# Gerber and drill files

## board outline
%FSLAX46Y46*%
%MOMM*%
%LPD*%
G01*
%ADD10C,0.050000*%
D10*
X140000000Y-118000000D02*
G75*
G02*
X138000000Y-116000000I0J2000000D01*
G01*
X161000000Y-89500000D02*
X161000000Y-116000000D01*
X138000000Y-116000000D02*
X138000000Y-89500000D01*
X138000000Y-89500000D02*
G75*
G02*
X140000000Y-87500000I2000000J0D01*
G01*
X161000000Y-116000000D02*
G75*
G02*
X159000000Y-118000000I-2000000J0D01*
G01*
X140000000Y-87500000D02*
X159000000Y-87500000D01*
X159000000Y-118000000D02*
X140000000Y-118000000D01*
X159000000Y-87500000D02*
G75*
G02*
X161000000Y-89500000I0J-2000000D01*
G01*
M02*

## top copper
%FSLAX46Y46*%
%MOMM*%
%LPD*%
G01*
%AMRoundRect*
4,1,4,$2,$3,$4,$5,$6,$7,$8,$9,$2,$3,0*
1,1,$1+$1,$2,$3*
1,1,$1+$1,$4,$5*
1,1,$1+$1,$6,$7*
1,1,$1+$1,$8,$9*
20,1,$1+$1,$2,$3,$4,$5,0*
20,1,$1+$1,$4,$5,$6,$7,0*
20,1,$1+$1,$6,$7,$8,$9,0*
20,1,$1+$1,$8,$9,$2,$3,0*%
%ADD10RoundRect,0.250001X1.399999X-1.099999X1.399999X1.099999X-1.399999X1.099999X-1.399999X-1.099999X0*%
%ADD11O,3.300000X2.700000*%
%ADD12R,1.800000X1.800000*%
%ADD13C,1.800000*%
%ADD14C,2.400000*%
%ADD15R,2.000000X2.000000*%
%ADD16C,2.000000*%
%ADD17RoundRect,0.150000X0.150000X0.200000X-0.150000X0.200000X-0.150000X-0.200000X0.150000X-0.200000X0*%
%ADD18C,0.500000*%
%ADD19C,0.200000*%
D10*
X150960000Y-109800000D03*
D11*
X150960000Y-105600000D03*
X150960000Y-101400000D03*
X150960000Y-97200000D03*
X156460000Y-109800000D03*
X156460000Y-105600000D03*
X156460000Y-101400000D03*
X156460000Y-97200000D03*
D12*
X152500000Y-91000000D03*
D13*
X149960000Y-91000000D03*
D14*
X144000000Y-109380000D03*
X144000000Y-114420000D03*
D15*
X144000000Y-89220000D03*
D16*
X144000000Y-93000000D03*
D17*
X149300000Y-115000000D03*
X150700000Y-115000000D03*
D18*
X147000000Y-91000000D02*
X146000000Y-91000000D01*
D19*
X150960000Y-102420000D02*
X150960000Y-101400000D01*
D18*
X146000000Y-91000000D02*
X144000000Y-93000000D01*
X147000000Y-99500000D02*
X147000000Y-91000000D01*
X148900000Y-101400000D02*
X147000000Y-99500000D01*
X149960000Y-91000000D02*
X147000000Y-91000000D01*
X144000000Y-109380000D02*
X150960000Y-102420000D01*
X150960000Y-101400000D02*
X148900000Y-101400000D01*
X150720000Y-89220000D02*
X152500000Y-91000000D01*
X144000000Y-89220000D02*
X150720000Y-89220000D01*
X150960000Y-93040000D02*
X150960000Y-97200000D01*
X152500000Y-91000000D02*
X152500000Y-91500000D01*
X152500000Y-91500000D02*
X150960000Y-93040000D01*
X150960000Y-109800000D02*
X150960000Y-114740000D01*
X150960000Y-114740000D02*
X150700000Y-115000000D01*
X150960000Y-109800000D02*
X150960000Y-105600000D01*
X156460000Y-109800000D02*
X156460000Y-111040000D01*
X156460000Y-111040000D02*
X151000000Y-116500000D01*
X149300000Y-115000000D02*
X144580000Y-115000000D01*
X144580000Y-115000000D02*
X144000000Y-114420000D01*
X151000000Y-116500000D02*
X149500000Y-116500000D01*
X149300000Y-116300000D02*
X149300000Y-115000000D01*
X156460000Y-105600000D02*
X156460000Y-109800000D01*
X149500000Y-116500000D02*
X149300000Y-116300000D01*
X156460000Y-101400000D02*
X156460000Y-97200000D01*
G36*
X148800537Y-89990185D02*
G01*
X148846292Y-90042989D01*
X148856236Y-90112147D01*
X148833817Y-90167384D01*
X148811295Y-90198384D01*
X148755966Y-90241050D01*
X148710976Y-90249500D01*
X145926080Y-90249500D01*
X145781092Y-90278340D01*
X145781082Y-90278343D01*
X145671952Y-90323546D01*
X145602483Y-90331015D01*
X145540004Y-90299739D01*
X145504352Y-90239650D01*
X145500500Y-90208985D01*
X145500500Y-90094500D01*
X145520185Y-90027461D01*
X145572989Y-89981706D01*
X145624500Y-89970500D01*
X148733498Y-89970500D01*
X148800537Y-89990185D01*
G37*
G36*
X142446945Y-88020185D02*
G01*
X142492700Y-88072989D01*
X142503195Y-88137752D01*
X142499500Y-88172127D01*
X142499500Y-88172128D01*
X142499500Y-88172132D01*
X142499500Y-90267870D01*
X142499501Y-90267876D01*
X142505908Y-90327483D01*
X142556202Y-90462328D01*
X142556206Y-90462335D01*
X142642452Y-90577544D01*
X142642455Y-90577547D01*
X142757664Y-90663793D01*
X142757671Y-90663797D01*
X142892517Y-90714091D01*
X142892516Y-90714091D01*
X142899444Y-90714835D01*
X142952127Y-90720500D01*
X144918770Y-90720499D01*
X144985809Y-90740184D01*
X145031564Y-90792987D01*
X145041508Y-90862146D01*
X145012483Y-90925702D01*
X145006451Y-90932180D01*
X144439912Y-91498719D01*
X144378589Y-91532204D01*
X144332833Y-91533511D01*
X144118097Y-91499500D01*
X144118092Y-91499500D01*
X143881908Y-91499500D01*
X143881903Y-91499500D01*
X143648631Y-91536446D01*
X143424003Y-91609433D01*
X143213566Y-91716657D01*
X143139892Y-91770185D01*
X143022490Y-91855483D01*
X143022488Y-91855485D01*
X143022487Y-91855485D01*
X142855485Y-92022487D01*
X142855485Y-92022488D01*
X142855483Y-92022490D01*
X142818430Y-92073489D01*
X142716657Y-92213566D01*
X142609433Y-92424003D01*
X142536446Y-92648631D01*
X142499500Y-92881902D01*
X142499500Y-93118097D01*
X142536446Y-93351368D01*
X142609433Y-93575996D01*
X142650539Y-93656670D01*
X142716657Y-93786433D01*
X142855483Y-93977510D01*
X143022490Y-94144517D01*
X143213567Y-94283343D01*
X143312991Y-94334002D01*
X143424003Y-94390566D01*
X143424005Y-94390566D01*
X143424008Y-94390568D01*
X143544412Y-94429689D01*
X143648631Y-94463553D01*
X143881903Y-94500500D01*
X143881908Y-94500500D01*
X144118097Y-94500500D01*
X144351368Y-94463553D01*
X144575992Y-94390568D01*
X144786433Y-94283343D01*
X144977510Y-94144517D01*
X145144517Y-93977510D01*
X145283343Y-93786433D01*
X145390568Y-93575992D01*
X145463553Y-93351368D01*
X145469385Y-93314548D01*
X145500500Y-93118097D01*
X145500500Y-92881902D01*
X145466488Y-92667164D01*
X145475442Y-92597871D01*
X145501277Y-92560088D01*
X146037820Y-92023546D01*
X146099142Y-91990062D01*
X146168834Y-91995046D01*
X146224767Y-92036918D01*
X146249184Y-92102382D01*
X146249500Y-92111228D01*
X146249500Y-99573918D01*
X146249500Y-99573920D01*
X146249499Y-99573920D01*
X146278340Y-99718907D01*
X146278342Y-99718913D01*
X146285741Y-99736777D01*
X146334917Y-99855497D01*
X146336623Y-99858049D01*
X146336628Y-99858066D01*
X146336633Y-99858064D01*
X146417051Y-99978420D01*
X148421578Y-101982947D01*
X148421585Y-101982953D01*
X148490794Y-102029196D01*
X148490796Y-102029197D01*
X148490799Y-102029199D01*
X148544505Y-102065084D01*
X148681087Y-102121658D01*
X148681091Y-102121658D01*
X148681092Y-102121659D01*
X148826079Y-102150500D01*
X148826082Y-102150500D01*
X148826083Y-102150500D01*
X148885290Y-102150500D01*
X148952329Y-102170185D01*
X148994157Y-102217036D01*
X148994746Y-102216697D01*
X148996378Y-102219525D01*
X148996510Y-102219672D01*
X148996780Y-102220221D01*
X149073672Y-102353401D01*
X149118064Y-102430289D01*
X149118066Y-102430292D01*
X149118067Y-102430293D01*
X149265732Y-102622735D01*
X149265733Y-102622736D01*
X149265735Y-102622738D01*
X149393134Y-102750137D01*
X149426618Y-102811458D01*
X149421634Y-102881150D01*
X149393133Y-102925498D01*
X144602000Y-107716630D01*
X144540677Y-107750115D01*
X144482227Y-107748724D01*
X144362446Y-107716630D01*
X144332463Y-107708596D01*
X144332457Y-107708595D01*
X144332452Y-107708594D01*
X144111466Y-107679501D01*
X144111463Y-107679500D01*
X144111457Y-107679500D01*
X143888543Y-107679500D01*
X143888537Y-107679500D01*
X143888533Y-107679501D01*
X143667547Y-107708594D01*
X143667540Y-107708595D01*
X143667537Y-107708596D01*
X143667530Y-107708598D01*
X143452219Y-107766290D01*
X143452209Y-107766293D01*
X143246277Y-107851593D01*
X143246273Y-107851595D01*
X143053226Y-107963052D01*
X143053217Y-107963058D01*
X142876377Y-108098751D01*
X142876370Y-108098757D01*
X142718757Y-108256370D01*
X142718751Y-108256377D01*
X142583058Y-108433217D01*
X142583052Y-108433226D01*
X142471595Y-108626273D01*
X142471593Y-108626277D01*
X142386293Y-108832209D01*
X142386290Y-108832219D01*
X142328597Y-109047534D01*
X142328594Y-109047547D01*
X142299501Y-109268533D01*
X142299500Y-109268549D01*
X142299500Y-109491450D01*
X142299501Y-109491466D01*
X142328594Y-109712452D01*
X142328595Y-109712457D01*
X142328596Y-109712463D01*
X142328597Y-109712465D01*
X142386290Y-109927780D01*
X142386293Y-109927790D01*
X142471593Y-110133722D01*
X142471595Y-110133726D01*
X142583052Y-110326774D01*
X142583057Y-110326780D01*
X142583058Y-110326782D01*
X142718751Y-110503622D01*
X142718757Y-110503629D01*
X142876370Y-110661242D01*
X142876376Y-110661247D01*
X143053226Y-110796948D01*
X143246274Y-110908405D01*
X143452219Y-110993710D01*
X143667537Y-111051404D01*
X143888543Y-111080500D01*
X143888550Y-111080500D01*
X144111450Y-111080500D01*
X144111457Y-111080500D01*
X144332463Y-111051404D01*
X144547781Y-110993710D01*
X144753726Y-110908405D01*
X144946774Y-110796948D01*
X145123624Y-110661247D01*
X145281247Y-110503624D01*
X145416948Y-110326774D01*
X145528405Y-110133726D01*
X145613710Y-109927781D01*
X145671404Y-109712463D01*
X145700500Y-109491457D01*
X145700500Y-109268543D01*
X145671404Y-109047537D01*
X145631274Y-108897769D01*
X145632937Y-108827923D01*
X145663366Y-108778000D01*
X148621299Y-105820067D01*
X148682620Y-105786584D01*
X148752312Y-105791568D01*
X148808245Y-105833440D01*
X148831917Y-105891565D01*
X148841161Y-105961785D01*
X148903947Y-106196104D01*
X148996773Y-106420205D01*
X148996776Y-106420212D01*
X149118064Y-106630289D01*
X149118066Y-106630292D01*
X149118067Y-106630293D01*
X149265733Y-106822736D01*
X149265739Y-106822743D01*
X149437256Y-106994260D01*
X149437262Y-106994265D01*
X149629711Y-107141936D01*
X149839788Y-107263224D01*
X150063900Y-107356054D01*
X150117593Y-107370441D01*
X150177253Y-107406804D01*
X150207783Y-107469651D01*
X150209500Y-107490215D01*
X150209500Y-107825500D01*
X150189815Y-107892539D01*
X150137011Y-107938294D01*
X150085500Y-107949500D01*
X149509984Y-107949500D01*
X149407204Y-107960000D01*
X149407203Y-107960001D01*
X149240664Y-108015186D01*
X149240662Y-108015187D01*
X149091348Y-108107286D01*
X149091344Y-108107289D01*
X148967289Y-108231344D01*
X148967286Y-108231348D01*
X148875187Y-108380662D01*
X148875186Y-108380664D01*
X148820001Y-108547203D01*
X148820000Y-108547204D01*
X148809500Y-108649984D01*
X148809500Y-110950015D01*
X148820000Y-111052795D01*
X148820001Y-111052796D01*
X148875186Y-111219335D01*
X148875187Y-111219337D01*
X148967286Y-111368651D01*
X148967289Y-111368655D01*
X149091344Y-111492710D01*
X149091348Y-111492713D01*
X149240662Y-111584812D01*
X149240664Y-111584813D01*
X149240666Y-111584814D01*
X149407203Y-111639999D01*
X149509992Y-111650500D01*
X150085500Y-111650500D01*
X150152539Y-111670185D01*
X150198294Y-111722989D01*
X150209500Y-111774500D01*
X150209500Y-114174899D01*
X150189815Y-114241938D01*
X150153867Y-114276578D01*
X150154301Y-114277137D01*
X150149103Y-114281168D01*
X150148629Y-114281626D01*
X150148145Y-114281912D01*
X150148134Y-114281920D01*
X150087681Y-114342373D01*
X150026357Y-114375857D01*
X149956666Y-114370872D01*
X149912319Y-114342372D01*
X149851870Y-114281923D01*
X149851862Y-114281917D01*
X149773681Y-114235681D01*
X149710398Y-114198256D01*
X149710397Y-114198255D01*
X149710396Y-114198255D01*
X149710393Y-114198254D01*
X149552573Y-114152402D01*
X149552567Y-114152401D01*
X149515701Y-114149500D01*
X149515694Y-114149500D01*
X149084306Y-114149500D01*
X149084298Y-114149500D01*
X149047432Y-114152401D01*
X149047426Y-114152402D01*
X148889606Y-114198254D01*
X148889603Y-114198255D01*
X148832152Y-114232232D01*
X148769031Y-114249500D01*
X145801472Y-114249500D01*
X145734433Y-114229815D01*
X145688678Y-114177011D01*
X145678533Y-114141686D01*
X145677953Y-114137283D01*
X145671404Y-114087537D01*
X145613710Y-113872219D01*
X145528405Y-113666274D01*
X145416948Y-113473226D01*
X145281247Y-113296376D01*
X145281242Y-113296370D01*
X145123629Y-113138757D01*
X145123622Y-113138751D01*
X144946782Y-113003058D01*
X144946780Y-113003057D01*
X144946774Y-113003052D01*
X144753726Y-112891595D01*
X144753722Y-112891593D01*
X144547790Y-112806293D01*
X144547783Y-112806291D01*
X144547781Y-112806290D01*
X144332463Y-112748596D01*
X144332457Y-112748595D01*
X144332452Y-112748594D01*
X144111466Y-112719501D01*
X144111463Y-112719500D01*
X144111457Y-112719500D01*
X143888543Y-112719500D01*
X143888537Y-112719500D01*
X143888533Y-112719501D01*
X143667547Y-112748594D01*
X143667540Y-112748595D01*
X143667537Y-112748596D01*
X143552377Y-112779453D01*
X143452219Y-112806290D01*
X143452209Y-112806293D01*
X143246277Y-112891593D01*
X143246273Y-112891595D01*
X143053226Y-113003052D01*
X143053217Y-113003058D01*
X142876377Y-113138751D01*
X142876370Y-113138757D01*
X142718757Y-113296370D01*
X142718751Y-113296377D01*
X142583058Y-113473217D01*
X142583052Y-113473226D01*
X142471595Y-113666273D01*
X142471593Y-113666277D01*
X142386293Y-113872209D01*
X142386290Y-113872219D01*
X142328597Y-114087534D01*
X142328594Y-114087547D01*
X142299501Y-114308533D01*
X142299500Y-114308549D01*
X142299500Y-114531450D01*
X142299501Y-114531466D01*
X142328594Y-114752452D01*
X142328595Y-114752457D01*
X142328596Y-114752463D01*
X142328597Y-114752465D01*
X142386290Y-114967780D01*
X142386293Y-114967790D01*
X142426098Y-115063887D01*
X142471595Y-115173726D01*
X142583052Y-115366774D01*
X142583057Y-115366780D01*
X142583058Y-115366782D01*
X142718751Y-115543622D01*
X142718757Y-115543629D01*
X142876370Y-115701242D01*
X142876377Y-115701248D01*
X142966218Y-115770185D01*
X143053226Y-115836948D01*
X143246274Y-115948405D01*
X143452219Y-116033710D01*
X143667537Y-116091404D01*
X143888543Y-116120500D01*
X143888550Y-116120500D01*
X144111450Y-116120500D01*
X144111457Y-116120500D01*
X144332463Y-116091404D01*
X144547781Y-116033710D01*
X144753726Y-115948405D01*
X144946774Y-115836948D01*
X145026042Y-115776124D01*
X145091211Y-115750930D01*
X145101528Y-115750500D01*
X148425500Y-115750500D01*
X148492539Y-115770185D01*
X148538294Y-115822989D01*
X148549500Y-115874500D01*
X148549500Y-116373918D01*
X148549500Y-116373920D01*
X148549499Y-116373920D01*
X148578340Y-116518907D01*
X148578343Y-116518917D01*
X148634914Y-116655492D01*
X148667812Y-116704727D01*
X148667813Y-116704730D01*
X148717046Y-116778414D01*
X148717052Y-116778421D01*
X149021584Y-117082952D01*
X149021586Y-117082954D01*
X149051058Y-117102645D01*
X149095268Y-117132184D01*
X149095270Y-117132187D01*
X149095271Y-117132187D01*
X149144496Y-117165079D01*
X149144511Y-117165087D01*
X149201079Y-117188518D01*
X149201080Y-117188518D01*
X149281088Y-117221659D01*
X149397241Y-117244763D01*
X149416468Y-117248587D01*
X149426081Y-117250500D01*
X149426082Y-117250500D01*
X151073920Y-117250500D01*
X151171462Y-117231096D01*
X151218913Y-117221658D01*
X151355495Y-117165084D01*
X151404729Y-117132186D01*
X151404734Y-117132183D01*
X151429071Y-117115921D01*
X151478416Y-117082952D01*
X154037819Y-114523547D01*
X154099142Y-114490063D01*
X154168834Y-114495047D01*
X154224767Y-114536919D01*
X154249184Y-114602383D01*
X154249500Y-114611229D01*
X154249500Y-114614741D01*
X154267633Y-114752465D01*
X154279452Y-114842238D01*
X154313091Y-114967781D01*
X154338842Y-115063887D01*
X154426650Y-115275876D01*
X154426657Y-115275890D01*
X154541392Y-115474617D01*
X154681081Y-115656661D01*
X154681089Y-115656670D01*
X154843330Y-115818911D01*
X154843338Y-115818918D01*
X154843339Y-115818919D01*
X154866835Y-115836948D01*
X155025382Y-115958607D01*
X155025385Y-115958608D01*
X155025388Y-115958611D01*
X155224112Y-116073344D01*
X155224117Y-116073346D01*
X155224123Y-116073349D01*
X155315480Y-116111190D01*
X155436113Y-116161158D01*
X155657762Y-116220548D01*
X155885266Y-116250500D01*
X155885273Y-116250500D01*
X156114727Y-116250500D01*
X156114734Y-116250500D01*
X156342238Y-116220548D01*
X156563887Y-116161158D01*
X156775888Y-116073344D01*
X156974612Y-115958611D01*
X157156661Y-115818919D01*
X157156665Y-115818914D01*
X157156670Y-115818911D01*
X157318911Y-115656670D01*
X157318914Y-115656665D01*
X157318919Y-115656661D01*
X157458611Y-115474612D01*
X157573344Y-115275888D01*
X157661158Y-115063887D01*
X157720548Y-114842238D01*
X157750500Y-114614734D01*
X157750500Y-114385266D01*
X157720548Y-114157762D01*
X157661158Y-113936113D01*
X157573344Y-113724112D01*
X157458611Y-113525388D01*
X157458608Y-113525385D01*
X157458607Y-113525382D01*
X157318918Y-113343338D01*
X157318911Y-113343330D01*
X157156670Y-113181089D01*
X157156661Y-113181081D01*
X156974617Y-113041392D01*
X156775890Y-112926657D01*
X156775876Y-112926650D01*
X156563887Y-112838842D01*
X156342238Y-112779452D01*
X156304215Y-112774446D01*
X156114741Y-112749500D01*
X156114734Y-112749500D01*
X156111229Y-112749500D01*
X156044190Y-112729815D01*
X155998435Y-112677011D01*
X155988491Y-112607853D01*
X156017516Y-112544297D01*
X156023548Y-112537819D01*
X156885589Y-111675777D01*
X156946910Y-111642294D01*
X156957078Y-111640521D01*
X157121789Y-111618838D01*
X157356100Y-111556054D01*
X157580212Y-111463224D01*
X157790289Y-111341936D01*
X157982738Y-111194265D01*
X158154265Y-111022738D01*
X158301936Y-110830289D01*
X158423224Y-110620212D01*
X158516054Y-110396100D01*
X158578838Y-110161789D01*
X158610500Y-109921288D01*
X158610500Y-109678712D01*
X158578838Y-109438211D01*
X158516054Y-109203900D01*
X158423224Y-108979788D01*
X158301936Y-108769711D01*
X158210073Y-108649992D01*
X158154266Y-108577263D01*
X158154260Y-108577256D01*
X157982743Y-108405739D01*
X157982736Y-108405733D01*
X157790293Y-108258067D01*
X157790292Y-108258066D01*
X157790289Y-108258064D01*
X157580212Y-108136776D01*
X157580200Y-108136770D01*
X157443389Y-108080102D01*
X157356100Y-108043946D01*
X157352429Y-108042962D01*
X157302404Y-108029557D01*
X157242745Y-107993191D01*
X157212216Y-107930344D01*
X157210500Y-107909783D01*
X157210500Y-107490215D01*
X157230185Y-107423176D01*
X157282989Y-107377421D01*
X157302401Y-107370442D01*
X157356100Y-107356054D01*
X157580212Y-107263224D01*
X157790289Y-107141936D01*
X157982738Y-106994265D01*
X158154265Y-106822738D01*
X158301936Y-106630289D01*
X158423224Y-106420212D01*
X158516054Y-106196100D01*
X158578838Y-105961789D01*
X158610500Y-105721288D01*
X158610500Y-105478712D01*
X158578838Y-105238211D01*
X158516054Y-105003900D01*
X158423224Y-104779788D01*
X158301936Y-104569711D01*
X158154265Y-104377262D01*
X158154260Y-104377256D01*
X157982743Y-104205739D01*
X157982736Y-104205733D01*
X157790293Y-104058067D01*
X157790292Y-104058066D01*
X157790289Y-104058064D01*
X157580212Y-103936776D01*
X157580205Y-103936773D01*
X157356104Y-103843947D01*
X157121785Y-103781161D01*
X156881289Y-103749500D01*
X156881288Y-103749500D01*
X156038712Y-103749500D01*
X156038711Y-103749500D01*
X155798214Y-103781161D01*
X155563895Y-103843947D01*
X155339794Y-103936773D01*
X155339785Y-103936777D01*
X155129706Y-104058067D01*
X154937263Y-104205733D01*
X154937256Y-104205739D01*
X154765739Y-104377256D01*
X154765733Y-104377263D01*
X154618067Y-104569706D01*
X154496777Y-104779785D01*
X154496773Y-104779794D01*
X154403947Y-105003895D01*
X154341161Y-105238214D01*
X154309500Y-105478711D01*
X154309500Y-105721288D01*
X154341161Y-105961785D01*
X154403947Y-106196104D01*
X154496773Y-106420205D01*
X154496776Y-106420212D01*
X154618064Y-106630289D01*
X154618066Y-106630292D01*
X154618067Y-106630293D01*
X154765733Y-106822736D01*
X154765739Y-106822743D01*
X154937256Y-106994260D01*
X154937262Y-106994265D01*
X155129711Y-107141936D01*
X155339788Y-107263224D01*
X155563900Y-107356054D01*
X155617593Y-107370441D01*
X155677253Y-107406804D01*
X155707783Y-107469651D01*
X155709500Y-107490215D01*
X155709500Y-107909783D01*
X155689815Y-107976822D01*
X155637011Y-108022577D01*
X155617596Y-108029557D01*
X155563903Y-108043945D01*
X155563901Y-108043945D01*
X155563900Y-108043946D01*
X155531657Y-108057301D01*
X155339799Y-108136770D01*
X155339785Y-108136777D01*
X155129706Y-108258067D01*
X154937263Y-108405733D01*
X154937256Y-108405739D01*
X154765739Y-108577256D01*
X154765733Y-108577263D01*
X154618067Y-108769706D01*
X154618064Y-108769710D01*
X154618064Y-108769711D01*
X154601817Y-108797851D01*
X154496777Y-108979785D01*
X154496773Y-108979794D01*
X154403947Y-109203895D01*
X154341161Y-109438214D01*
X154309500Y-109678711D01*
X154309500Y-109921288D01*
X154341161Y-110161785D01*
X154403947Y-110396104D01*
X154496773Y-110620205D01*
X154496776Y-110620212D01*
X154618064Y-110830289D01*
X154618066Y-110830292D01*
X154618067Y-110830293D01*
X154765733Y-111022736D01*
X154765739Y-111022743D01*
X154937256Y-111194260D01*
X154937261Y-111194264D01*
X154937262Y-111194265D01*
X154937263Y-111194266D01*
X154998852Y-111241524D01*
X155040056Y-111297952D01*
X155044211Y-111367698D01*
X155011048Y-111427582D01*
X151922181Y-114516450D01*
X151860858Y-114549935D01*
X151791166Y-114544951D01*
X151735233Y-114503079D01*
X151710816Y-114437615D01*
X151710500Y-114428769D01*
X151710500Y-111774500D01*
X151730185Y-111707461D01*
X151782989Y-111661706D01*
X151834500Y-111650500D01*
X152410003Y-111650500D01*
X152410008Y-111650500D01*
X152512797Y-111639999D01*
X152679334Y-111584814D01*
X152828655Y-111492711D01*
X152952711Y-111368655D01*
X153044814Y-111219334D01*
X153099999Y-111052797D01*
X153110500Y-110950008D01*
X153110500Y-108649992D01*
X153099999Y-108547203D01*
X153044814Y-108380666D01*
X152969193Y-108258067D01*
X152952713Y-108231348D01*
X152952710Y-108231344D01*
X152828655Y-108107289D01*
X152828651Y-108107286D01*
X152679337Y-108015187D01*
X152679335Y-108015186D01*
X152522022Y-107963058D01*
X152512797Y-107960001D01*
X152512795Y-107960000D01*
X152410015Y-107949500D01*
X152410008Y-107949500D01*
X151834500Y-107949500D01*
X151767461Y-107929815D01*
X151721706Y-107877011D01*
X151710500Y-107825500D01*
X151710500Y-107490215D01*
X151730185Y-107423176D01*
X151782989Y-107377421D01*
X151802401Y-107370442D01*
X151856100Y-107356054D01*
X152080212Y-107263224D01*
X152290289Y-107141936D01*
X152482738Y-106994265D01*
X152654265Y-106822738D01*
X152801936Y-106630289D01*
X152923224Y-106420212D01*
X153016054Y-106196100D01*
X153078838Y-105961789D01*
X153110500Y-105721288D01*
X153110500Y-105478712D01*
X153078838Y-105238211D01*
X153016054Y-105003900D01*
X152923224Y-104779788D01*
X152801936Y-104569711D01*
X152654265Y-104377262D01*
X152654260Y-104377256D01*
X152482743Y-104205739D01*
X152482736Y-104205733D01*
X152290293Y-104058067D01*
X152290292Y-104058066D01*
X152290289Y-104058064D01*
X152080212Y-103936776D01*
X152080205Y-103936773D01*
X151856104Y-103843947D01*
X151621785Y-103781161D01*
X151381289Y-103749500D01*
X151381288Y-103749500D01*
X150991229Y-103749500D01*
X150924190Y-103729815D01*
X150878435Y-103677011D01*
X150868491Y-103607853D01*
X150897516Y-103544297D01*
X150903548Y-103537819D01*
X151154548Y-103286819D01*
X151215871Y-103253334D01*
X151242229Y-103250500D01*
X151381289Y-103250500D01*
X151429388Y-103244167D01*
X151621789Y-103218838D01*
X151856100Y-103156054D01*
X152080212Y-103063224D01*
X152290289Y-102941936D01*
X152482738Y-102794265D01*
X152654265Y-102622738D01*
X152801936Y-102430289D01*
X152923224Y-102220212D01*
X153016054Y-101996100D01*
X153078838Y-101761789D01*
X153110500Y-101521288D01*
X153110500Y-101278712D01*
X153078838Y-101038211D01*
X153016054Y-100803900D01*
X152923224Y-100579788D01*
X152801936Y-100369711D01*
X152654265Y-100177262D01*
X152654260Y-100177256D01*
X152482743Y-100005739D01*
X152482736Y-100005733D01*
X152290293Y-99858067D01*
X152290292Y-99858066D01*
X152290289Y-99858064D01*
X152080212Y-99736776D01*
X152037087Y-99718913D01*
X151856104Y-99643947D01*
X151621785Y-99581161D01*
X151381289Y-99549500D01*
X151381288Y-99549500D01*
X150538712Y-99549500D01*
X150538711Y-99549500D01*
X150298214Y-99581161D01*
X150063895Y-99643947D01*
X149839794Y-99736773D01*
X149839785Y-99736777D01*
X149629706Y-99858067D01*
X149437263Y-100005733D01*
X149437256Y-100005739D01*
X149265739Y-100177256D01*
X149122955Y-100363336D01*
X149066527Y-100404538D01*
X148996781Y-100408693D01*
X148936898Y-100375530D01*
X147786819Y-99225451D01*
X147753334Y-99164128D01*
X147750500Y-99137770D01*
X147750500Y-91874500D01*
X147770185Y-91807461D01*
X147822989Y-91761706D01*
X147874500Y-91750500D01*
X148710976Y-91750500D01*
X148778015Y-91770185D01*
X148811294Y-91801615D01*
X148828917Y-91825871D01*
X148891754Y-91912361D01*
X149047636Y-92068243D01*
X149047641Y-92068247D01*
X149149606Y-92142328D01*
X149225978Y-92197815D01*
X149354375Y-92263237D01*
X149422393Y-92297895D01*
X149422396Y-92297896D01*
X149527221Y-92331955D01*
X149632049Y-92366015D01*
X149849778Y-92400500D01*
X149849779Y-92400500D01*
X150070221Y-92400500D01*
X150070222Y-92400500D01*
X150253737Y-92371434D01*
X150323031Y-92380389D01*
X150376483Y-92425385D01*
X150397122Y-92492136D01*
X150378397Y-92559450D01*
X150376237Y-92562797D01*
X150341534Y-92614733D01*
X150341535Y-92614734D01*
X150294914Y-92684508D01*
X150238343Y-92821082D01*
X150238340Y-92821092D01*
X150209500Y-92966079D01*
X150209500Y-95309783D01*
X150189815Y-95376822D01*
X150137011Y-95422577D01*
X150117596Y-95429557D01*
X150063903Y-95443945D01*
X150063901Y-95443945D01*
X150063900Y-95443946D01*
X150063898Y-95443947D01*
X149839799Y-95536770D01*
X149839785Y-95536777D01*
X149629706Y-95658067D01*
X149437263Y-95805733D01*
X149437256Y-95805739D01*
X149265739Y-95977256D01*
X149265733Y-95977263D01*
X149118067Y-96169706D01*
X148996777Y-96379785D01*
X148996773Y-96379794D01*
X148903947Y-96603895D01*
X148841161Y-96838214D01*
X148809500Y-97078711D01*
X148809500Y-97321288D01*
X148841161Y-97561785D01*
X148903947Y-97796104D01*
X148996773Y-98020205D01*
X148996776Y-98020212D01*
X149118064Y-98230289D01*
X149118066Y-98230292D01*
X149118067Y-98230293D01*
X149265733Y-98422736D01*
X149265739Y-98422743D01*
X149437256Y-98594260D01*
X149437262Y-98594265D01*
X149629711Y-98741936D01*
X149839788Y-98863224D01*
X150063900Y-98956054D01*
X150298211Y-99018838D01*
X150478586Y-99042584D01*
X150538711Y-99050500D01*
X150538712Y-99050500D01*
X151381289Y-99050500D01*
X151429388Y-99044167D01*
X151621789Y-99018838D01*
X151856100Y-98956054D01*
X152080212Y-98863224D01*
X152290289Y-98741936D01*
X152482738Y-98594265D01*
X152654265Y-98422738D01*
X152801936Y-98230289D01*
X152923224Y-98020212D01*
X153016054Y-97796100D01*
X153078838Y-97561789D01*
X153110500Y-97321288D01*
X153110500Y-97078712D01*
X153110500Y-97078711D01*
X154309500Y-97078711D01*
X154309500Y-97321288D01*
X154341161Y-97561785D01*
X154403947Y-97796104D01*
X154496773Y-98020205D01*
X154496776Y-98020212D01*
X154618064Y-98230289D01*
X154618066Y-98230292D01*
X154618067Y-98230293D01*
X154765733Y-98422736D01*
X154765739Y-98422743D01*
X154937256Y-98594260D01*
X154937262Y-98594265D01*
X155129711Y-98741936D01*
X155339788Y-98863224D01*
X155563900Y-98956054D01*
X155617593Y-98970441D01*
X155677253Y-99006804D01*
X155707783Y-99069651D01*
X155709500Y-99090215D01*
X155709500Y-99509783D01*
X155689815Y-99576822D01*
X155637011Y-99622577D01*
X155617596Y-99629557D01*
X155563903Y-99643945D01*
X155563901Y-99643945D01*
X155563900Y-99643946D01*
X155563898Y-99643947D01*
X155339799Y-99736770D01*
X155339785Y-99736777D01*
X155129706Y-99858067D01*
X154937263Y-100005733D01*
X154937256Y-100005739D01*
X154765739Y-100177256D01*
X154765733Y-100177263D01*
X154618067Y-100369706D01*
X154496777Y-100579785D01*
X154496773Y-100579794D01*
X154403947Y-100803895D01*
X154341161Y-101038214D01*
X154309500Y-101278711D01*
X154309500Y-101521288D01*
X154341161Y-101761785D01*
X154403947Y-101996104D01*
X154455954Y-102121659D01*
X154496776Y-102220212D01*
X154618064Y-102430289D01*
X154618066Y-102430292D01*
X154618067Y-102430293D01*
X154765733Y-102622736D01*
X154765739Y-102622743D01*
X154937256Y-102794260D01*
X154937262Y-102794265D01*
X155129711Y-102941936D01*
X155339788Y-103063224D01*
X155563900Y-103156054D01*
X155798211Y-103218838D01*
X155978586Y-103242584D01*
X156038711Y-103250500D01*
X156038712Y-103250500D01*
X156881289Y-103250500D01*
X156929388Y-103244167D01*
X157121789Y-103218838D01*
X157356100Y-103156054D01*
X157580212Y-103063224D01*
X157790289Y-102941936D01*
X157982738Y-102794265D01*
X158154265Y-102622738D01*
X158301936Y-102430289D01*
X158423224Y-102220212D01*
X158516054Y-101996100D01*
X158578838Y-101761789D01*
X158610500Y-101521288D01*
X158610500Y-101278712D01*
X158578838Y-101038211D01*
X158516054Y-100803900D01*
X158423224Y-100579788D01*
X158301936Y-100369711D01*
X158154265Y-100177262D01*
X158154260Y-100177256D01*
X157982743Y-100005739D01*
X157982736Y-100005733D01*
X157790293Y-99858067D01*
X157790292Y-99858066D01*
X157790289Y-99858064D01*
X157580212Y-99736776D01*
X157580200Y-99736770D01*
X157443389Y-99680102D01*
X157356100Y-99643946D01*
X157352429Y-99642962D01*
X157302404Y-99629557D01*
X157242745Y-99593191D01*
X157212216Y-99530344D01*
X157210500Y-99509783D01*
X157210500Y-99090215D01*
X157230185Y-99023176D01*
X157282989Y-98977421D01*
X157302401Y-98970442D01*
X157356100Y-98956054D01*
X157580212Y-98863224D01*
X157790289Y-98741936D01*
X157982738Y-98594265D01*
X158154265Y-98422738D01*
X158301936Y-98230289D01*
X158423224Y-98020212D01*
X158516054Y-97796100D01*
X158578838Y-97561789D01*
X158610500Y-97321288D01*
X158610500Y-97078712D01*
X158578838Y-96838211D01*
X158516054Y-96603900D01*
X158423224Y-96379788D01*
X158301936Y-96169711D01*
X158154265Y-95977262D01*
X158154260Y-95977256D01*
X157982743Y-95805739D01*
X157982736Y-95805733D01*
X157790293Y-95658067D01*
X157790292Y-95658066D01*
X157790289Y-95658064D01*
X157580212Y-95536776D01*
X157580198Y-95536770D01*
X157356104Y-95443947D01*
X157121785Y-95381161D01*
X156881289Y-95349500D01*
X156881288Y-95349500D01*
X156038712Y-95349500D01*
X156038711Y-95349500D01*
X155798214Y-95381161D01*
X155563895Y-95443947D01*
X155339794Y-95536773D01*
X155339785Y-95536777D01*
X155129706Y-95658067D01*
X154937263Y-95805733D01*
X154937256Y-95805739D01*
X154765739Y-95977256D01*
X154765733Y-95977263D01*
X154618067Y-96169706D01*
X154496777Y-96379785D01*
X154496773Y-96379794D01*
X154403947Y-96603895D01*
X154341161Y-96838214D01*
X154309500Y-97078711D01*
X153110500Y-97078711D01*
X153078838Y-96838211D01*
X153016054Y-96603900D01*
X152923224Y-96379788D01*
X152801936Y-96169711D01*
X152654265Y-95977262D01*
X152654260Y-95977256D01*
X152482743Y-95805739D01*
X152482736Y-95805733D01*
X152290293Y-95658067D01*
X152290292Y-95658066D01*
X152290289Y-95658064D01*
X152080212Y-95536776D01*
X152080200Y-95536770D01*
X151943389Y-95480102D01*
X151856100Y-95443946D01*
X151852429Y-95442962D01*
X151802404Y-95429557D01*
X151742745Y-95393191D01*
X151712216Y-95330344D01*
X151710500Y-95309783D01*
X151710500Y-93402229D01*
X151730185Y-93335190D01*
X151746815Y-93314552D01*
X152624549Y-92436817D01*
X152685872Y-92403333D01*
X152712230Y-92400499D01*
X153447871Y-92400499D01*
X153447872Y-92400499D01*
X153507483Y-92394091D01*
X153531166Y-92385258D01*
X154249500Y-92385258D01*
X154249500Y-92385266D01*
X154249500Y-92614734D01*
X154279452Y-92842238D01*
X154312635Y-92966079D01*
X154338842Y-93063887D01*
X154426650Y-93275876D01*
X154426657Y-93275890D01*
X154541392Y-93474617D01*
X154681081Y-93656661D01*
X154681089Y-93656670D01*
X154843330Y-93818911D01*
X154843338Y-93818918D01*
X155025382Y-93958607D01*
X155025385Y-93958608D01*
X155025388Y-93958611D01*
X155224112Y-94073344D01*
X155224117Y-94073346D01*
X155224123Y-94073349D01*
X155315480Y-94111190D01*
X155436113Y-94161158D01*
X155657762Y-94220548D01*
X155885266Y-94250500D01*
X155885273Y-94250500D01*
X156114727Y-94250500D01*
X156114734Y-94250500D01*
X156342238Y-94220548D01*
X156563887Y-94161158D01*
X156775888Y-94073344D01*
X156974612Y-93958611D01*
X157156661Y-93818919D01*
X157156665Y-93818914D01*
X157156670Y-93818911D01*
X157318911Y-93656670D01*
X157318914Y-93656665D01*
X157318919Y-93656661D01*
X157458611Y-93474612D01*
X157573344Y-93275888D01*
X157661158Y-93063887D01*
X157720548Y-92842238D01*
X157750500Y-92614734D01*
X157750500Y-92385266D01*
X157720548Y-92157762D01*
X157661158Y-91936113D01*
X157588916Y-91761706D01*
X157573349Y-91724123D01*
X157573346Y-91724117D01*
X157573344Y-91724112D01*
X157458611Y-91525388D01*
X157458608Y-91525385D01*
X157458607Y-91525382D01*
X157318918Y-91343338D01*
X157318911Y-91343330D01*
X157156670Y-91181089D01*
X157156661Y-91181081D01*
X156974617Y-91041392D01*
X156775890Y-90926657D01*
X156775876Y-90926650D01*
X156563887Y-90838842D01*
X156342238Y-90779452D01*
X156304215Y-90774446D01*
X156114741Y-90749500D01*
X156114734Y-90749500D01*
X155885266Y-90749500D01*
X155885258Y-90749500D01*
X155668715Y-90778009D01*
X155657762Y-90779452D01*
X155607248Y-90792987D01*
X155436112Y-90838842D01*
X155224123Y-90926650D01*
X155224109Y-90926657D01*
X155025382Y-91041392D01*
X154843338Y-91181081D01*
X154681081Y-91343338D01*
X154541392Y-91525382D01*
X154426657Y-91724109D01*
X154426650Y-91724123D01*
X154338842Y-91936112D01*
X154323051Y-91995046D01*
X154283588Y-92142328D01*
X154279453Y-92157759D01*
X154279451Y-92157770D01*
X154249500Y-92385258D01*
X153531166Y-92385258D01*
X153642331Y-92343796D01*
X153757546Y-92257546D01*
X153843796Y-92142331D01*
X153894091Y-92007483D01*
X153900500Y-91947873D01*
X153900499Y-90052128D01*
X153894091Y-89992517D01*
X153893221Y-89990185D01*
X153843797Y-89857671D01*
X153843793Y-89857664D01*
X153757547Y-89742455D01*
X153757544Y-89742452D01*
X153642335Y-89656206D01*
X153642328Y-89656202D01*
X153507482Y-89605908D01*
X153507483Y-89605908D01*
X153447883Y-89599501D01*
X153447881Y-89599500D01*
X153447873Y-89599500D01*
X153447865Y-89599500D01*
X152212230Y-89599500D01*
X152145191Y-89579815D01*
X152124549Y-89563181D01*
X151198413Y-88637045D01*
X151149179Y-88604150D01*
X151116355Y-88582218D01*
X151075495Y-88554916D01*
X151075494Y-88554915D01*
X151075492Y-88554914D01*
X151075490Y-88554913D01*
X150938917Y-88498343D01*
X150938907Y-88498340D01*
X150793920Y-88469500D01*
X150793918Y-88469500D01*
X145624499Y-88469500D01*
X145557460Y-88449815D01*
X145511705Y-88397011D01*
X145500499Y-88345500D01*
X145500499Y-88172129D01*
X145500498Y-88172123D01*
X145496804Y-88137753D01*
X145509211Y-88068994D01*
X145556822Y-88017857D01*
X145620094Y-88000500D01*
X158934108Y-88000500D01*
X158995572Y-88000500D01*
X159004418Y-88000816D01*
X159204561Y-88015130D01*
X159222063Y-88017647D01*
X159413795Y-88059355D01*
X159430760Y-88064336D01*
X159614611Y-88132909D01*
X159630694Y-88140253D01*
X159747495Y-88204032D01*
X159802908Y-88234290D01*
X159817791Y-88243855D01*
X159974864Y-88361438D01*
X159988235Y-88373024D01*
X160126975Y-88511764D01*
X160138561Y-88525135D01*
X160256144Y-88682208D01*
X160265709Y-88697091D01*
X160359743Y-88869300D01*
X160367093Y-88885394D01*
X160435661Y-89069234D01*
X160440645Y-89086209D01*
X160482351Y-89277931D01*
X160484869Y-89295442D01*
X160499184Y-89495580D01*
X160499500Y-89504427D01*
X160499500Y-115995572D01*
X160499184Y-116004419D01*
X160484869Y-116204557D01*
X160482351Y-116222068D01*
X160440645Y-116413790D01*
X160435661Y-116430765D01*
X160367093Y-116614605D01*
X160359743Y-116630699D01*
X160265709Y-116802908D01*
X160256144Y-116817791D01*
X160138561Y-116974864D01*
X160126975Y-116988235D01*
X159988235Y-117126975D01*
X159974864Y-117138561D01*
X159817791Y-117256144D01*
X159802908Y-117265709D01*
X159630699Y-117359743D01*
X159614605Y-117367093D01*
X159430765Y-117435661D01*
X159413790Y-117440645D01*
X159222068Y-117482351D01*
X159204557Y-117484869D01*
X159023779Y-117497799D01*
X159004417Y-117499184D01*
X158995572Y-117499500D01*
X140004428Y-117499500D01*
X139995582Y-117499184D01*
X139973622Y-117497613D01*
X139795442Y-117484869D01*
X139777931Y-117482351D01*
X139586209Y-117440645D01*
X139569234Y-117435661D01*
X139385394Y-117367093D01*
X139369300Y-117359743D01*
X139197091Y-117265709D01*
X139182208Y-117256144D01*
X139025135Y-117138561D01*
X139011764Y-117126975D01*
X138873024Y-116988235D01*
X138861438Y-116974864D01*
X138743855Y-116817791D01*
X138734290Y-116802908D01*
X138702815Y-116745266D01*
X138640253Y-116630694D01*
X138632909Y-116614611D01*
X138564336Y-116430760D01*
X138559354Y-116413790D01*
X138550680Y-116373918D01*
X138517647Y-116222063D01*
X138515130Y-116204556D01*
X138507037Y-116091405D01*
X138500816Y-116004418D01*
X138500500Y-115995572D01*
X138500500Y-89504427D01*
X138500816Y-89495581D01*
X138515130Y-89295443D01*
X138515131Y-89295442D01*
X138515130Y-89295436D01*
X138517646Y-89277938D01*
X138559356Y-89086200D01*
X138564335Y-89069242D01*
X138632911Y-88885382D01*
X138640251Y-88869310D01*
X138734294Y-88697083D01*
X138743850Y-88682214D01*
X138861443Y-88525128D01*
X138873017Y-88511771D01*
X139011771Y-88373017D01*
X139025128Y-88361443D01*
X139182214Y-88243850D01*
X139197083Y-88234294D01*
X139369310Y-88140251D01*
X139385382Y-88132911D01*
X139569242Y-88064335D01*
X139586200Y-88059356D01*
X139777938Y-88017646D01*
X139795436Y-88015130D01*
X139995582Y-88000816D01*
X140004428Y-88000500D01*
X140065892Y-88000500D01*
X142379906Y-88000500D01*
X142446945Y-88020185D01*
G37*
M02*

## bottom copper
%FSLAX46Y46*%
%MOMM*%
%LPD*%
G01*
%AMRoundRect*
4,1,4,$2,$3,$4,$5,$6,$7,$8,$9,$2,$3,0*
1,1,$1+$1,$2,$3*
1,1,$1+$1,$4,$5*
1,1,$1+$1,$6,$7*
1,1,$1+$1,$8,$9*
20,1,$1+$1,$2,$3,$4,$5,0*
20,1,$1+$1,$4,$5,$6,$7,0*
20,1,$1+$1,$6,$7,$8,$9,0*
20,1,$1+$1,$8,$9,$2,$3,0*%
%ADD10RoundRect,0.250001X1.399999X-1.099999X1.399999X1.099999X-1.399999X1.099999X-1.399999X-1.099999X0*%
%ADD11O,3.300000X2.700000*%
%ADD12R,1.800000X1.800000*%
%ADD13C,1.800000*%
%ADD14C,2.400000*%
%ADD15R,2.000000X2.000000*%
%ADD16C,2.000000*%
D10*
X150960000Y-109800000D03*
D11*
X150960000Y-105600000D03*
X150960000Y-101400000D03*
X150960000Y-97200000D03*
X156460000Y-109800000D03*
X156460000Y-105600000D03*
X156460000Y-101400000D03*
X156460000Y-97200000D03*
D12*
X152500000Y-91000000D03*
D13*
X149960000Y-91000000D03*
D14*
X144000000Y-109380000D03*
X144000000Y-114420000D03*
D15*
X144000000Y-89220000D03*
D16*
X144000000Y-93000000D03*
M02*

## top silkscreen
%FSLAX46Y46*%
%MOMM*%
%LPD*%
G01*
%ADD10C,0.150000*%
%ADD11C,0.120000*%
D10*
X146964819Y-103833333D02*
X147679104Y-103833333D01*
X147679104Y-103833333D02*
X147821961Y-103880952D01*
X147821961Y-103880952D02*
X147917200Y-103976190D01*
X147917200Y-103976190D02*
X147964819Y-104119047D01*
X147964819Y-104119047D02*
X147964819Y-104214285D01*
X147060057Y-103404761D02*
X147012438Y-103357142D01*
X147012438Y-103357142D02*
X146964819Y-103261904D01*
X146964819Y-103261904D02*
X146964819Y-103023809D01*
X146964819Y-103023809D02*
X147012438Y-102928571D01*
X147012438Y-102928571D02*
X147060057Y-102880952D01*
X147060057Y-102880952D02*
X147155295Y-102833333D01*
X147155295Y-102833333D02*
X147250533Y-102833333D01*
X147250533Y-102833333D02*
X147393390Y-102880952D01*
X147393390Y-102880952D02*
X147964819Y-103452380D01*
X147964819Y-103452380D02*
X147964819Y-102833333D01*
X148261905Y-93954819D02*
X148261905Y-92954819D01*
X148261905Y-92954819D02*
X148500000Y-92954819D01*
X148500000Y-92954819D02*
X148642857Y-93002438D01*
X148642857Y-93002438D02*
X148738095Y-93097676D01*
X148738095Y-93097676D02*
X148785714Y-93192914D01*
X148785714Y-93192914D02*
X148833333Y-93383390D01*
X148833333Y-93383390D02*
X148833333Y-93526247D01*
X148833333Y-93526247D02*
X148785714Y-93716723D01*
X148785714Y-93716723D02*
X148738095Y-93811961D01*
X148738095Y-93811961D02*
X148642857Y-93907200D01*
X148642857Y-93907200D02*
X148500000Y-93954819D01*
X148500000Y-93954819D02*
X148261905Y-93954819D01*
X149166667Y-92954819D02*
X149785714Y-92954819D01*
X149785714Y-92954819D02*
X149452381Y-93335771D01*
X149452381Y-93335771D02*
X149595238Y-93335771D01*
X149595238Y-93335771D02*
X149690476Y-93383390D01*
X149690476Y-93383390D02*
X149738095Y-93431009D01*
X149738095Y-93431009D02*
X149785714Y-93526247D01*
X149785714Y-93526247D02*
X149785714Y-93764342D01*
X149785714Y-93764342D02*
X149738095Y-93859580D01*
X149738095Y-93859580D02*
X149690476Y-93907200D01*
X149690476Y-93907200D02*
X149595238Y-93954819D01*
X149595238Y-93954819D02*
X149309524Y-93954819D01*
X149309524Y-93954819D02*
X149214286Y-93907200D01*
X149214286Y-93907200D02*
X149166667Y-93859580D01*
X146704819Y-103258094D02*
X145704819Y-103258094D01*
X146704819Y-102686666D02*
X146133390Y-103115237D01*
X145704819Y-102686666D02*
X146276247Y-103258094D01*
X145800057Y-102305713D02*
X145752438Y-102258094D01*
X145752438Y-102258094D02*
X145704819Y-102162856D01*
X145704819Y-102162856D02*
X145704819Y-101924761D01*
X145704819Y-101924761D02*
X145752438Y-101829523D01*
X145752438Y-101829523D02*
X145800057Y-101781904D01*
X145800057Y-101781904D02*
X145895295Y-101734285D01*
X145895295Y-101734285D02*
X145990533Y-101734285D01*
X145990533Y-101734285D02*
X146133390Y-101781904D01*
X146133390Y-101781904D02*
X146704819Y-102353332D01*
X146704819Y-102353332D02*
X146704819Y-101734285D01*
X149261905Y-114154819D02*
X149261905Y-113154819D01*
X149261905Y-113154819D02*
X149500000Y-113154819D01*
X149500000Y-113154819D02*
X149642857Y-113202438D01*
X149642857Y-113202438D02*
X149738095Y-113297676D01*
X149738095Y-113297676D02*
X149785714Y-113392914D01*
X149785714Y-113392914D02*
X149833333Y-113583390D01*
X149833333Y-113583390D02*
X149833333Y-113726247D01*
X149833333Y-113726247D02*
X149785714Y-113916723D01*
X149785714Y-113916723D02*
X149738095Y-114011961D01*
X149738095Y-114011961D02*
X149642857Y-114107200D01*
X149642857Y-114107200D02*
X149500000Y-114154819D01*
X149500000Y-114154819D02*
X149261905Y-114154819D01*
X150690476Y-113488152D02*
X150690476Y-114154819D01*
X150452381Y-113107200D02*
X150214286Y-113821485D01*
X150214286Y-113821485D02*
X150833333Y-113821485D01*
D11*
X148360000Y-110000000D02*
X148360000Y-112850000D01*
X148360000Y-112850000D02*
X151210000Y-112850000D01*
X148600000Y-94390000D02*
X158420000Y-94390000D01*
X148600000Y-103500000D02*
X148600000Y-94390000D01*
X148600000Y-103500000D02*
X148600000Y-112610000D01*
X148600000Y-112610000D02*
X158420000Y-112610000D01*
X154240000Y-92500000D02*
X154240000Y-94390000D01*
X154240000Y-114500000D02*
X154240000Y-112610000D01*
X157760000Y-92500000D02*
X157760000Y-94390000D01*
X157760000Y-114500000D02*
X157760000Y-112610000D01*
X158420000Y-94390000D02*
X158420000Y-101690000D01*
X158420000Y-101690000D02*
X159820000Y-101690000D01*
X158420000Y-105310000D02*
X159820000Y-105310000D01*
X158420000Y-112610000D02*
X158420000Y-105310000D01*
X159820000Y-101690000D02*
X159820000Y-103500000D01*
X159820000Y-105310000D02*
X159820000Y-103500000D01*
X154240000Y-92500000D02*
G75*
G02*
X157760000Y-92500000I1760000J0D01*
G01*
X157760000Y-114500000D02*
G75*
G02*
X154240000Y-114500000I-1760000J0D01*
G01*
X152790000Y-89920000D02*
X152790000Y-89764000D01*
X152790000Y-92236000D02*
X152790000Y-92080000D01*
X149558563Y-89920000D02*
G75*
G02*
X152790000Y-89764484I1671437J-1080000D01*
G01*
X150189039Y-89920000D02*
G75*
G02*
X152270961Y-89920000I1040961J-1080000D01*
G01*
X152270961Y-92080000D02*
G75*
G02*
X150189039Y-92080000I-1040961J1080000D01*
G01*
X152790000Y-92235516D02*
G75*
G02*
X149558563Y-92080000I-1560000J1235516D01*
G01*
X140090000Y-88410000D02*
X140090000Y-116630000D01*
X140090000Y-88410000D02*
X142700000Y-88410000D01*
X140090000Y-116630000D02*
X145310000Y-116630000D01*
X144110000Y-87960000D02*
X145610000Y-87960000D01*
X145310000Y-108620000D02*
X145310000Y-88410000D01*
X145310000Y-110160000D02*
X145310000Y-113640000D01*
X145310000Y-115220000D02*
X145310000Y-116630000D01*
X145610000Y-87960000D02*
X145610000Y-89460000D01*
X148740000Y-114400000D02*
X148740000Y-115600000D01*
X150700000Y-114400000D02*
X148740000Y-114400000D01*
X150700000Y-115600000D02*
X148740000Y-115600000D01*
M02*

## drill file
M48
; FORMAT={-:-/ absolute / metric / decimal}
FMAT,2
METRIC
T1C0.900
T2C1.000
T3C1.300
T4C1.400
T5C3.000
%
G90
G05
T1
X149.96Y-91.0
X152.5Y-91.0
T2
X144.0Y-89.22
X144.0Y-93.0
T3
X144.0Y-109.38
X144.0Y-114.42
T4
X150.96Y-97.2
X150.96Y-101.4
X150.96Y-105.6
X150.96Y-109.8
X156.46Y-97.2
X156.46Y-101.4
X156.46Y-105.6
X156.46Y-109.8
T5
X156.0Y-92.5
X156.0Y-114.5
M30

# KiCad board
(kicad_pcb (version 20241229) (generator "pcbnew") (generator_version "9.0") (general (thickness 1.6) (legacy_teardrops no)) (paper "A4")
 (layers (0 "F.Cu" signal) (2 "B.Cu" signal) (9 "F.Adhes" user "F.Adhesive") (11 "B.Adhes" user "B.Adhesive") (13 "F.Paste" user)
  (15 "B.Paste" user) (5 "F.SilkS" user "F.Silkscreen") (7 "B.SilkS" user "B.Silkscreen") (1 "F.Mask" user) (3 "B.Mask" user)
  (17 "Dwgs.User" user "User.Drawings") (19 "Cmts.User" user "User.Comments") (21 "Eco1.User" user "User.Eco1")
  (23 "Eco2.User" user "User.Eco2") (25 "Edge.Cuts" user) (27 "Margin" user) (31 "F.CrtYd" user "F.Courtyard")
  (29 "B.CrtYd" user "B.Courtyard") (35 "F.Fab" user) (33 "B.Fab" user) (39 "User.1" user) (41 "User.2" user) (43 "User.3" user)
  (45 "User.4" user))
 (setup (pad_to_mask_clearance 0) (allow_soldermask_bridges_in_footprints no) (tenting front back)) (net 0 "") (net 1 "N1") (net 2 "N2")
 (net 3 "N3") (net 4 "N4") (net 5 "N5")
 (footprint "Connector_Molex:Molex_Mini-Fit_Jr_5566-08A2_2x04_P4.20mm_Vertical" (layer "F.Cu") (at 150.96 109.8 90)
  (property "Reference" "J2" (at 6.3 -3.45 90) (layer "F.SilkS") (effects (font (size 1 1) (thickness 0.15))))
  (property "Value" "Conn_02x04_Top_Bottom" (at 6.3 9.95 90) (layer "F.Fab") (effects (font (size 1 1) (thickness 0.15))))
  (fp_line (start -0.2 -2.6) (end -3.05 -2.6) (stroke (width 0.12) (type solid)) (layer "F.SilkS"))
  (fp_line (start -3.05 -2.6) (end -3.05 0.25) (stroke (width 0.12) (type solid)) (layer "F.SilkS"))
  (fp_line (start 15.41 -2.36) (end 15.41 7.46) (stroke (width 0.12) (type solid)) (layer "F.SilkS"))
  (fp_line (start 6.3 -2.36) (end 15.41 -2.36) (stroke (width 0.12) (type solid)) (layer "F.SilkS"))
  (fp_line (start 6.3 -2.36) (end -2.81 -2.36) (stroke (width 0.12) (type solid)) (layer "F.SilkS"))
  (fp_line (start -2.81 -2.36) (end -2.81 7.46) (stroke (width 0.12) (type solid)) (layer "F.SilkS"))
  (fp_line (start 17.3 3.28) (end 15.41 3.28) (stroke (width 0.12) (type solid)) (layer "F.SilkS"))
  (fp_line (start -4.7 3.28) (end -2.81 3.28) (stroke (width 0.12) (type solid)) (layer "F.SilkS"))
  (fp_line (start 17.3 6.8) (end 15.41 6.8) (stroke (width 0.12) (type solid)) (layer "F.SilkS"))
  (fp_line (start -4.7 6.8) (end -2.81 6.8) (stroke (width 0.12) (type solid)) (layer "F.SilkS"))
  (fp_line (start 15.41 7.46) (end 8.11 7.46) (stroke (width 0.12) (type solid)) (layer "F.SilkS"))
  (fp_line (start 8.11 7.46) (end 8.11 8.86) (stroke (width 0.12) (type solid)) (layer "F.SilkS"))
  (fp_line (start 4.49 7.46) (end 4.49 8.86) (stroke (width 0.12) (type solid)) (layer "F.SilkS"))
  (fp_line (start -2.81 7.46) (end 4.49 7.46) (stroke (width 0.12) (type solid)) (layer "F.SilkS"))
  (fp_line (start 8.11 8.86) (end 6.3 8.86) (stroke (width 0.12) (type solid)) (layer "F.SilkS"))
  (fp_line (start 4.49 8.86) (end 6.3 8.86) (stroke (width 0.12) (type solid)) (layer "F.SilkS"))
  (fp_arc (start 17.3 3.28) (mid 19.06 5.04) (end 17.3 6.8) (stroke (width 0.12) (type solid)) (layer "F.SilkS"))
  (fp_arc (start -4.7 6.8) (mid -6.46 5.04) (end -4.7 3.28) (stroke (width 0.12) (type solid)) (layer "F.SilkS"))
  (pad "" np_thru_hole circle (at -4.7 5.04 90) (size 3 3) (drill 3) (layers "*.Cu" "*.Mask"))
  (pad "" np_thru_hole circle (at 17.3 5.04 90) (size 3 3) (drill 3) (layers "*.Cu" "*.Mask"))
  (pad "1" thru_hole roundrect (at 0 0 90) (size 2.7 3.3) (drill 1.4) (layers "*.Cu" "*.Mask") (remove_unused_layers no)
   (roundrect_rratio 0.092593) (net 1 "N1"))
  (pad "2" thru_hole oval (at 4.2 0 90) (size 2.7 3.3) (drill 1.4) (layers "*.Cu" "*.Mask") (remove_unused_layers no) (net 1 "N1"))
  (pad "3" thru_hole oval (at 8.4 0 90) (size 2.7 3.3) (drill 1.4) (layers "*.Cu" "*.Mask") (remove_unused_layers no) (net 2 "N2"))
  (pad "4" thru_hole oval (at 12.6 0 90) (size 2.7 3.3) (drill 1.4) (layers "*.Cu" "*.Mask") (remove_unused_layers no) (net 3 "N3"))
  (pad "5" thru_hole oval (at 0 5.5 90) (size 2.7 3.3) (drill 1.4) (layers "*.Cu" "*.Mask") (remove_unused_layers no) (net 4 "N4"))
  (pad "6" thru_hole oval (at 4.2 5.5 90) (size 2.7 3.3) (drill 1.4) (layers "*.Cu" "*.Mask") (remove_unused_layers no) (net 4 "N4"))
  (pad "7" thru_hole oval (at 8.4 5.5 90) (size 2.7 3.3) (drill 1.4) (layers "*.Cu" "*.Mask") (remove_unused_layers no) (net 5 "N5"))
  (pad "8" thru_hole oval (at 12.6 5.5 90) (size 2.7 3.3) (drill 1.4) (layers "*.Cu" "*.Mask") (remove_unused_layers no) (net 5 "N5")))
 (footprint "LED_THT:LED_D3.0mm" (layer "F.Cu") (at 152.5 91 180)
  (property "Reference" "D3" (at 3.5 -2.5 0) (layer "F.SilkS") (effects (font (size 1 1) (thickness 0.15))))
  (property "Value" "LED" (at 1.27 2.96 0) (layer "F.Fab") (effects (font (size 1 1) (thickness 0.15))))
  (fp_line (start -0.29 1.08) (end -0.29 1.236) (stroke (width 0.12) (type solid)) (layer "F.SilkS"))
  (fp_line (start -0.29 -1.236) (end -0.29 -1.08) (stroke (width 0.12) (type solid)) (layer "F.SilkS"))
  (fp_arc (start 2.941437 1.08) (mid 1.36566 1.987699) (end -0.29 1.235516) (stroke (width 0.12) (type solid)) (layer "F.SilkS"))
  (fp_arc (start 2.310961 1.08) (mid 1.27 1.5) (end 0.229039 1.08) (stroke (width 0.12) (type solid)) (layer "F.SilkS"))
  (fp_arc (start 0.229039 -1.08) (mid 1.27 -1.5) (end 2.310961 -1.08) (stroke (width 0.12) (type solid)) (layer "F.SilkS"))
  (fp_arc (start -0.29 -1.235516) (mid 1.36566 -1.987699) (end 2.941437 -1.08) (stroke (width 0.12) (type solid)) (layer "F.SilkS"))
  (pad "1" thru_hole rect (at 0 0 180) (size 1.8 1.8) (drill 0.9) (layers "*.Cu" "*.Mask") (remove_unused_layers no) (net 3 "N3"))
  (pad "2" thru_hole circle (at 2.54 0 180) (size 1.8 1.8) (drill 0.9) (layers "*.Cu" "*.Mask") (remove_unused_layers no) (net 2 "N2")))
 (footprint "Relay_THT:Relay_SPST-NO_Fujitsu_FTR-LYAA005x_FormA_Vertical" (layer "F.Cu") (at 144 89.22 -90)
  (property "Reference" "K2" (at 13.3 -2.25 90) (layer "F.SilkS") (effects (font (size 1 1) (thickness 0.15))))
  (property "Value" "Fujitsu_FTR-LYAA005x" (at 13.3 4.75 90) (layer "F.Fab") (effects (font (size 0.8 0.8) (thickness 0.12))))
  (fp_line (start -0.81 3.91) (end 27.41 3.91) (stroke (width 0.12) (type solid)) (layer "F.SilkS"))
  (fp_line (start -0.81 3.91) (end -0.81 1.3) (stroke (width 0.12) (type solid)) (layer "F.SilkS"))
  (fp_line (start 27.41 3.91) (end 27.41 -1.31) (stroke (width 0.12) (type solid)) (layer "F.SilkS"))
  (fp_line (start -1.26 -0.11) (end -1.26 -1.61) (stroke (width 0.12) (type solid)) (layer "F.SilkS"))
  (fp_line (start 19.4 -1.31) (end -0.81 -1.31) (stroke (width 0.12) (type solid)) (layer "F.SilkS"))
  (fp_line (start 20.94 -1.31) (end 24.42 -1.31) (stroke (width 0.12) (type solid)) (layer "F.SilkS"))
  (fp_line (start 26 -1.31) (end 27.41 -1.31) (stroke (width 0.12) (type solid)) (layer "F.SilkS"))
  (fp_line (start -1.26 -1.61) (end 0.24 -1.61) (stroke (width 0.12) (type solid)) (layer "F.SilkS"))
  (pad "13" thru_hole circle (at 20.16 0 270) (size 2.4 2.4) (drill 1.3) (layers "*.Cu" "*.Mask") (remove_unused_layers no) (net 2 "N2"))
  (pad "14" thru_hole circle (at 25.2 0 270) (size 2.4 2.4) (drill 1.3) (layers "*.Cu" "*.Mask") (remove_unused_layers no) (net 4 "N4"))
  (pad "A1" thru_hole rect (at 0 0 270) (size 2 2) (drill 1) (layers "*.Cu" "*.Mask") (remove_unused_layers no) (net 3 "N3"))
  (pad "A2" thru_hole circle (at 3.78 0 270) (size 2 2) (drill 1) (layers "*.Cu" "*.Mask") (remove_unused_layers no) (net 2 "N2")))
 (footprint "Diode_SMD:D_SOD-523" (layer "F.Cu") (at 150 115)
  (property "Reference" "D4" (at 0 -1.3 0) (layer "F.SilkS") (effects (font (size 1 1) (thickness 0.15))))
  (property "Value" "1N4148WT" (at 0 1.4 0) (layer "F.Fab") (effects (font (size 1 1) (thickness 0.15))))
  (fp_line (start -1.26 -0.6) (end -1.26 0.6) (stroke (width 0.12) (type solid)) (layer "F.SilkS"))
  (fp_line (start 0.7 -0.6) (end -1.26 -0.6) (stroke (width 0.12) (type solid)) (layer "F.SilkS"))
  (fp_line (start 0.7 0.6) (end -1.26 0.6) (stroke (width 0.12) (type solid)) (layer "F.SilkS"))
  (pad "1" smd roundrect (at -0.7 0 180) (size 0.6 0.7) (layers "F.Cu" "F.Mask" "F.Paste") (roundrect_rratio 0.25) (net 4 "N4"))
  (pad "2" smd roundrect (at 0.7 0 180) (size 0.6 0.7) (layers "F.Cu" "F.Mask" "F.Paste") (roundrect_rratio 0.25) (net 1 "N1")))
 (gr_arc (start 140 118) (mid 138.585786 117.414214) (end 138 116) (stroke (width 0.05) (type default)) (layer "Edge.Cuts"))
 (gr_line (start 161 89.5) (end 161 116) (stroke (width 0.05) (type default)) (layer "Edge.Cuts"))
 (gr_line (start 138 116) (end 138 89.5) (stroke (width 0.05) (type default)) (layer "Edge.Cuts"))
 (gr_arc (start 138 89.5) (mid 138.585786 88.085786) (end 140 87.5) (stroke (width 0.05) (type default)) (layer "Edge.Cuts"))
 (gr_arc (start 161 116) (mid 160.414214 117.414214) (end 159 118) (stroke (width 0.05) (type default)) (layer "Edge.Cuts"))
 (gr_line (start 140 87.5) (end 159 87.5) (stroke (width 0.05) (type default)) (layer "Edge.Cuts"))
 (gr_line (start 159 118) (end 140 118) (stroke (width 0.05) (type default)) (layer "Edge.Cuts"))
 (gr_arc (start 159 87.5) (mid 160.414214 88.085786) (end 161 89.5) (stroke (width 0.05) (type default)) (layer "Edge.Cuts"))
 (segment (start 147 91) (end 146 91) (width 0.5) (layer "F.Cu") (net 2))
 (segment (start 150.96 102.42) (end 150.96 101.4) (width 0.2) (layer "F.Cu") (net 2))
 (segment (start 146 91) (end 144 93) (width 0.5) (layer "F.Cu") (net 2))
 (segment (start 147 99.5) (end 147 91) (width 0.5) (layer "F.Cu") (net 2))
 (segment (start 148.9 101.4) (end 147 99.5) (width 0.5) (layer "F.Cu") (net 2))
 (segment (start 149.96 91) (end 147 91) (width 0.5) (layer "F.Cu") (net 2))
 (segment (start 144 109.38) (end 150.96 102.42) (width 0.5) (layer "F.Cu") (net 2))
 (segment (start 150.96 101.4) (end 148.9 101.4) (width 0.5) (layer "F.Cu") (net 2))
 (segment (start 150.72 89.22) (end 152.5 91) (width 0.5) (layer "F.Cu") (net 3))
 (segment (start 144 89.22) (end 150.72 89.22) (width 0.5) (layer "F.Cu") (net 3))
 (segment (start 150.96 93.04) (end 150.96 97.2) (width 0.5) (layer "F.Cu") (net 3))
 (segment (start 152.5 91) (end 152.5 91.5) (width 0.5) (layer "F.Cu") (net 3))
 (segment (start 152.5 91.5) (end 150.96 93.04) (width 0.5) (layer "F.Cu") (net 3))
 (segment (start 150.96 109.8) (end 150.96 114.74) (width 0.5) (layer "F.Cu") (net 1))
 (segment (start 150.96 114.74) (end 150.7 115) (width 0.5) (layer "F.Cu") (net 1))
 (segment (start 150.96 109.8) (end 150.96 105.6) (width 0.5) (layer "F.Cu") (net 1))
 (segment (start 156.46 109.8) (end 156.46 111.04) (width 0.5) (layer "F.Cu") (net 4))
 (segment (start 156.46 111.04) (end 151 116.5) (width 0.5) (layer "F.Cu") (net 4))
 (segment (start 149.3 115) (end 144.58 115) (width 0.5) (layer "F.Cu") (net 4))
 (segment (start 144.58 115) (end 144 114.42) (width 0.5) (layer "F.Cu") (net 4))
 (segment (start 151 116.5) (end 149.5 116.5) (width 0.5) (layer "F.Cu") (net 4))
 (segment (start 149.3 116.3) (end 149.3 115) (width 0.5) (layer "F.Cu") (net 4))
 (segment (start 156.46 105.6) (end 156.46 109.8) (width 0.5) (layer "F.Cu") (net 4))
 (segment (start 149.5 116.5) (end 149.3 116.3) (width 0.5) (layer "F.Cu") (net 4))
 (segment (start 156.46 101.4) (end 156.46 97.2) (width 0.5) (layer "F.Cu") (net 5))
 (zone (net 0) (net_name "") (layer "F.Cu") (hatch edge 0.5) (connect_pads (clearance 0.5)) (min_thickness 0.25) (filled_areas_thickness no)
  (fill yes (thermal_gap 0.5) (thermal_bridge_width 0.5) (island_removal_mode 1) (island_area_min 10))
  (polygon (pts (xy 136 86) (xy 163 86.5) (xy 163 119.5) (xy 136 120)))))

